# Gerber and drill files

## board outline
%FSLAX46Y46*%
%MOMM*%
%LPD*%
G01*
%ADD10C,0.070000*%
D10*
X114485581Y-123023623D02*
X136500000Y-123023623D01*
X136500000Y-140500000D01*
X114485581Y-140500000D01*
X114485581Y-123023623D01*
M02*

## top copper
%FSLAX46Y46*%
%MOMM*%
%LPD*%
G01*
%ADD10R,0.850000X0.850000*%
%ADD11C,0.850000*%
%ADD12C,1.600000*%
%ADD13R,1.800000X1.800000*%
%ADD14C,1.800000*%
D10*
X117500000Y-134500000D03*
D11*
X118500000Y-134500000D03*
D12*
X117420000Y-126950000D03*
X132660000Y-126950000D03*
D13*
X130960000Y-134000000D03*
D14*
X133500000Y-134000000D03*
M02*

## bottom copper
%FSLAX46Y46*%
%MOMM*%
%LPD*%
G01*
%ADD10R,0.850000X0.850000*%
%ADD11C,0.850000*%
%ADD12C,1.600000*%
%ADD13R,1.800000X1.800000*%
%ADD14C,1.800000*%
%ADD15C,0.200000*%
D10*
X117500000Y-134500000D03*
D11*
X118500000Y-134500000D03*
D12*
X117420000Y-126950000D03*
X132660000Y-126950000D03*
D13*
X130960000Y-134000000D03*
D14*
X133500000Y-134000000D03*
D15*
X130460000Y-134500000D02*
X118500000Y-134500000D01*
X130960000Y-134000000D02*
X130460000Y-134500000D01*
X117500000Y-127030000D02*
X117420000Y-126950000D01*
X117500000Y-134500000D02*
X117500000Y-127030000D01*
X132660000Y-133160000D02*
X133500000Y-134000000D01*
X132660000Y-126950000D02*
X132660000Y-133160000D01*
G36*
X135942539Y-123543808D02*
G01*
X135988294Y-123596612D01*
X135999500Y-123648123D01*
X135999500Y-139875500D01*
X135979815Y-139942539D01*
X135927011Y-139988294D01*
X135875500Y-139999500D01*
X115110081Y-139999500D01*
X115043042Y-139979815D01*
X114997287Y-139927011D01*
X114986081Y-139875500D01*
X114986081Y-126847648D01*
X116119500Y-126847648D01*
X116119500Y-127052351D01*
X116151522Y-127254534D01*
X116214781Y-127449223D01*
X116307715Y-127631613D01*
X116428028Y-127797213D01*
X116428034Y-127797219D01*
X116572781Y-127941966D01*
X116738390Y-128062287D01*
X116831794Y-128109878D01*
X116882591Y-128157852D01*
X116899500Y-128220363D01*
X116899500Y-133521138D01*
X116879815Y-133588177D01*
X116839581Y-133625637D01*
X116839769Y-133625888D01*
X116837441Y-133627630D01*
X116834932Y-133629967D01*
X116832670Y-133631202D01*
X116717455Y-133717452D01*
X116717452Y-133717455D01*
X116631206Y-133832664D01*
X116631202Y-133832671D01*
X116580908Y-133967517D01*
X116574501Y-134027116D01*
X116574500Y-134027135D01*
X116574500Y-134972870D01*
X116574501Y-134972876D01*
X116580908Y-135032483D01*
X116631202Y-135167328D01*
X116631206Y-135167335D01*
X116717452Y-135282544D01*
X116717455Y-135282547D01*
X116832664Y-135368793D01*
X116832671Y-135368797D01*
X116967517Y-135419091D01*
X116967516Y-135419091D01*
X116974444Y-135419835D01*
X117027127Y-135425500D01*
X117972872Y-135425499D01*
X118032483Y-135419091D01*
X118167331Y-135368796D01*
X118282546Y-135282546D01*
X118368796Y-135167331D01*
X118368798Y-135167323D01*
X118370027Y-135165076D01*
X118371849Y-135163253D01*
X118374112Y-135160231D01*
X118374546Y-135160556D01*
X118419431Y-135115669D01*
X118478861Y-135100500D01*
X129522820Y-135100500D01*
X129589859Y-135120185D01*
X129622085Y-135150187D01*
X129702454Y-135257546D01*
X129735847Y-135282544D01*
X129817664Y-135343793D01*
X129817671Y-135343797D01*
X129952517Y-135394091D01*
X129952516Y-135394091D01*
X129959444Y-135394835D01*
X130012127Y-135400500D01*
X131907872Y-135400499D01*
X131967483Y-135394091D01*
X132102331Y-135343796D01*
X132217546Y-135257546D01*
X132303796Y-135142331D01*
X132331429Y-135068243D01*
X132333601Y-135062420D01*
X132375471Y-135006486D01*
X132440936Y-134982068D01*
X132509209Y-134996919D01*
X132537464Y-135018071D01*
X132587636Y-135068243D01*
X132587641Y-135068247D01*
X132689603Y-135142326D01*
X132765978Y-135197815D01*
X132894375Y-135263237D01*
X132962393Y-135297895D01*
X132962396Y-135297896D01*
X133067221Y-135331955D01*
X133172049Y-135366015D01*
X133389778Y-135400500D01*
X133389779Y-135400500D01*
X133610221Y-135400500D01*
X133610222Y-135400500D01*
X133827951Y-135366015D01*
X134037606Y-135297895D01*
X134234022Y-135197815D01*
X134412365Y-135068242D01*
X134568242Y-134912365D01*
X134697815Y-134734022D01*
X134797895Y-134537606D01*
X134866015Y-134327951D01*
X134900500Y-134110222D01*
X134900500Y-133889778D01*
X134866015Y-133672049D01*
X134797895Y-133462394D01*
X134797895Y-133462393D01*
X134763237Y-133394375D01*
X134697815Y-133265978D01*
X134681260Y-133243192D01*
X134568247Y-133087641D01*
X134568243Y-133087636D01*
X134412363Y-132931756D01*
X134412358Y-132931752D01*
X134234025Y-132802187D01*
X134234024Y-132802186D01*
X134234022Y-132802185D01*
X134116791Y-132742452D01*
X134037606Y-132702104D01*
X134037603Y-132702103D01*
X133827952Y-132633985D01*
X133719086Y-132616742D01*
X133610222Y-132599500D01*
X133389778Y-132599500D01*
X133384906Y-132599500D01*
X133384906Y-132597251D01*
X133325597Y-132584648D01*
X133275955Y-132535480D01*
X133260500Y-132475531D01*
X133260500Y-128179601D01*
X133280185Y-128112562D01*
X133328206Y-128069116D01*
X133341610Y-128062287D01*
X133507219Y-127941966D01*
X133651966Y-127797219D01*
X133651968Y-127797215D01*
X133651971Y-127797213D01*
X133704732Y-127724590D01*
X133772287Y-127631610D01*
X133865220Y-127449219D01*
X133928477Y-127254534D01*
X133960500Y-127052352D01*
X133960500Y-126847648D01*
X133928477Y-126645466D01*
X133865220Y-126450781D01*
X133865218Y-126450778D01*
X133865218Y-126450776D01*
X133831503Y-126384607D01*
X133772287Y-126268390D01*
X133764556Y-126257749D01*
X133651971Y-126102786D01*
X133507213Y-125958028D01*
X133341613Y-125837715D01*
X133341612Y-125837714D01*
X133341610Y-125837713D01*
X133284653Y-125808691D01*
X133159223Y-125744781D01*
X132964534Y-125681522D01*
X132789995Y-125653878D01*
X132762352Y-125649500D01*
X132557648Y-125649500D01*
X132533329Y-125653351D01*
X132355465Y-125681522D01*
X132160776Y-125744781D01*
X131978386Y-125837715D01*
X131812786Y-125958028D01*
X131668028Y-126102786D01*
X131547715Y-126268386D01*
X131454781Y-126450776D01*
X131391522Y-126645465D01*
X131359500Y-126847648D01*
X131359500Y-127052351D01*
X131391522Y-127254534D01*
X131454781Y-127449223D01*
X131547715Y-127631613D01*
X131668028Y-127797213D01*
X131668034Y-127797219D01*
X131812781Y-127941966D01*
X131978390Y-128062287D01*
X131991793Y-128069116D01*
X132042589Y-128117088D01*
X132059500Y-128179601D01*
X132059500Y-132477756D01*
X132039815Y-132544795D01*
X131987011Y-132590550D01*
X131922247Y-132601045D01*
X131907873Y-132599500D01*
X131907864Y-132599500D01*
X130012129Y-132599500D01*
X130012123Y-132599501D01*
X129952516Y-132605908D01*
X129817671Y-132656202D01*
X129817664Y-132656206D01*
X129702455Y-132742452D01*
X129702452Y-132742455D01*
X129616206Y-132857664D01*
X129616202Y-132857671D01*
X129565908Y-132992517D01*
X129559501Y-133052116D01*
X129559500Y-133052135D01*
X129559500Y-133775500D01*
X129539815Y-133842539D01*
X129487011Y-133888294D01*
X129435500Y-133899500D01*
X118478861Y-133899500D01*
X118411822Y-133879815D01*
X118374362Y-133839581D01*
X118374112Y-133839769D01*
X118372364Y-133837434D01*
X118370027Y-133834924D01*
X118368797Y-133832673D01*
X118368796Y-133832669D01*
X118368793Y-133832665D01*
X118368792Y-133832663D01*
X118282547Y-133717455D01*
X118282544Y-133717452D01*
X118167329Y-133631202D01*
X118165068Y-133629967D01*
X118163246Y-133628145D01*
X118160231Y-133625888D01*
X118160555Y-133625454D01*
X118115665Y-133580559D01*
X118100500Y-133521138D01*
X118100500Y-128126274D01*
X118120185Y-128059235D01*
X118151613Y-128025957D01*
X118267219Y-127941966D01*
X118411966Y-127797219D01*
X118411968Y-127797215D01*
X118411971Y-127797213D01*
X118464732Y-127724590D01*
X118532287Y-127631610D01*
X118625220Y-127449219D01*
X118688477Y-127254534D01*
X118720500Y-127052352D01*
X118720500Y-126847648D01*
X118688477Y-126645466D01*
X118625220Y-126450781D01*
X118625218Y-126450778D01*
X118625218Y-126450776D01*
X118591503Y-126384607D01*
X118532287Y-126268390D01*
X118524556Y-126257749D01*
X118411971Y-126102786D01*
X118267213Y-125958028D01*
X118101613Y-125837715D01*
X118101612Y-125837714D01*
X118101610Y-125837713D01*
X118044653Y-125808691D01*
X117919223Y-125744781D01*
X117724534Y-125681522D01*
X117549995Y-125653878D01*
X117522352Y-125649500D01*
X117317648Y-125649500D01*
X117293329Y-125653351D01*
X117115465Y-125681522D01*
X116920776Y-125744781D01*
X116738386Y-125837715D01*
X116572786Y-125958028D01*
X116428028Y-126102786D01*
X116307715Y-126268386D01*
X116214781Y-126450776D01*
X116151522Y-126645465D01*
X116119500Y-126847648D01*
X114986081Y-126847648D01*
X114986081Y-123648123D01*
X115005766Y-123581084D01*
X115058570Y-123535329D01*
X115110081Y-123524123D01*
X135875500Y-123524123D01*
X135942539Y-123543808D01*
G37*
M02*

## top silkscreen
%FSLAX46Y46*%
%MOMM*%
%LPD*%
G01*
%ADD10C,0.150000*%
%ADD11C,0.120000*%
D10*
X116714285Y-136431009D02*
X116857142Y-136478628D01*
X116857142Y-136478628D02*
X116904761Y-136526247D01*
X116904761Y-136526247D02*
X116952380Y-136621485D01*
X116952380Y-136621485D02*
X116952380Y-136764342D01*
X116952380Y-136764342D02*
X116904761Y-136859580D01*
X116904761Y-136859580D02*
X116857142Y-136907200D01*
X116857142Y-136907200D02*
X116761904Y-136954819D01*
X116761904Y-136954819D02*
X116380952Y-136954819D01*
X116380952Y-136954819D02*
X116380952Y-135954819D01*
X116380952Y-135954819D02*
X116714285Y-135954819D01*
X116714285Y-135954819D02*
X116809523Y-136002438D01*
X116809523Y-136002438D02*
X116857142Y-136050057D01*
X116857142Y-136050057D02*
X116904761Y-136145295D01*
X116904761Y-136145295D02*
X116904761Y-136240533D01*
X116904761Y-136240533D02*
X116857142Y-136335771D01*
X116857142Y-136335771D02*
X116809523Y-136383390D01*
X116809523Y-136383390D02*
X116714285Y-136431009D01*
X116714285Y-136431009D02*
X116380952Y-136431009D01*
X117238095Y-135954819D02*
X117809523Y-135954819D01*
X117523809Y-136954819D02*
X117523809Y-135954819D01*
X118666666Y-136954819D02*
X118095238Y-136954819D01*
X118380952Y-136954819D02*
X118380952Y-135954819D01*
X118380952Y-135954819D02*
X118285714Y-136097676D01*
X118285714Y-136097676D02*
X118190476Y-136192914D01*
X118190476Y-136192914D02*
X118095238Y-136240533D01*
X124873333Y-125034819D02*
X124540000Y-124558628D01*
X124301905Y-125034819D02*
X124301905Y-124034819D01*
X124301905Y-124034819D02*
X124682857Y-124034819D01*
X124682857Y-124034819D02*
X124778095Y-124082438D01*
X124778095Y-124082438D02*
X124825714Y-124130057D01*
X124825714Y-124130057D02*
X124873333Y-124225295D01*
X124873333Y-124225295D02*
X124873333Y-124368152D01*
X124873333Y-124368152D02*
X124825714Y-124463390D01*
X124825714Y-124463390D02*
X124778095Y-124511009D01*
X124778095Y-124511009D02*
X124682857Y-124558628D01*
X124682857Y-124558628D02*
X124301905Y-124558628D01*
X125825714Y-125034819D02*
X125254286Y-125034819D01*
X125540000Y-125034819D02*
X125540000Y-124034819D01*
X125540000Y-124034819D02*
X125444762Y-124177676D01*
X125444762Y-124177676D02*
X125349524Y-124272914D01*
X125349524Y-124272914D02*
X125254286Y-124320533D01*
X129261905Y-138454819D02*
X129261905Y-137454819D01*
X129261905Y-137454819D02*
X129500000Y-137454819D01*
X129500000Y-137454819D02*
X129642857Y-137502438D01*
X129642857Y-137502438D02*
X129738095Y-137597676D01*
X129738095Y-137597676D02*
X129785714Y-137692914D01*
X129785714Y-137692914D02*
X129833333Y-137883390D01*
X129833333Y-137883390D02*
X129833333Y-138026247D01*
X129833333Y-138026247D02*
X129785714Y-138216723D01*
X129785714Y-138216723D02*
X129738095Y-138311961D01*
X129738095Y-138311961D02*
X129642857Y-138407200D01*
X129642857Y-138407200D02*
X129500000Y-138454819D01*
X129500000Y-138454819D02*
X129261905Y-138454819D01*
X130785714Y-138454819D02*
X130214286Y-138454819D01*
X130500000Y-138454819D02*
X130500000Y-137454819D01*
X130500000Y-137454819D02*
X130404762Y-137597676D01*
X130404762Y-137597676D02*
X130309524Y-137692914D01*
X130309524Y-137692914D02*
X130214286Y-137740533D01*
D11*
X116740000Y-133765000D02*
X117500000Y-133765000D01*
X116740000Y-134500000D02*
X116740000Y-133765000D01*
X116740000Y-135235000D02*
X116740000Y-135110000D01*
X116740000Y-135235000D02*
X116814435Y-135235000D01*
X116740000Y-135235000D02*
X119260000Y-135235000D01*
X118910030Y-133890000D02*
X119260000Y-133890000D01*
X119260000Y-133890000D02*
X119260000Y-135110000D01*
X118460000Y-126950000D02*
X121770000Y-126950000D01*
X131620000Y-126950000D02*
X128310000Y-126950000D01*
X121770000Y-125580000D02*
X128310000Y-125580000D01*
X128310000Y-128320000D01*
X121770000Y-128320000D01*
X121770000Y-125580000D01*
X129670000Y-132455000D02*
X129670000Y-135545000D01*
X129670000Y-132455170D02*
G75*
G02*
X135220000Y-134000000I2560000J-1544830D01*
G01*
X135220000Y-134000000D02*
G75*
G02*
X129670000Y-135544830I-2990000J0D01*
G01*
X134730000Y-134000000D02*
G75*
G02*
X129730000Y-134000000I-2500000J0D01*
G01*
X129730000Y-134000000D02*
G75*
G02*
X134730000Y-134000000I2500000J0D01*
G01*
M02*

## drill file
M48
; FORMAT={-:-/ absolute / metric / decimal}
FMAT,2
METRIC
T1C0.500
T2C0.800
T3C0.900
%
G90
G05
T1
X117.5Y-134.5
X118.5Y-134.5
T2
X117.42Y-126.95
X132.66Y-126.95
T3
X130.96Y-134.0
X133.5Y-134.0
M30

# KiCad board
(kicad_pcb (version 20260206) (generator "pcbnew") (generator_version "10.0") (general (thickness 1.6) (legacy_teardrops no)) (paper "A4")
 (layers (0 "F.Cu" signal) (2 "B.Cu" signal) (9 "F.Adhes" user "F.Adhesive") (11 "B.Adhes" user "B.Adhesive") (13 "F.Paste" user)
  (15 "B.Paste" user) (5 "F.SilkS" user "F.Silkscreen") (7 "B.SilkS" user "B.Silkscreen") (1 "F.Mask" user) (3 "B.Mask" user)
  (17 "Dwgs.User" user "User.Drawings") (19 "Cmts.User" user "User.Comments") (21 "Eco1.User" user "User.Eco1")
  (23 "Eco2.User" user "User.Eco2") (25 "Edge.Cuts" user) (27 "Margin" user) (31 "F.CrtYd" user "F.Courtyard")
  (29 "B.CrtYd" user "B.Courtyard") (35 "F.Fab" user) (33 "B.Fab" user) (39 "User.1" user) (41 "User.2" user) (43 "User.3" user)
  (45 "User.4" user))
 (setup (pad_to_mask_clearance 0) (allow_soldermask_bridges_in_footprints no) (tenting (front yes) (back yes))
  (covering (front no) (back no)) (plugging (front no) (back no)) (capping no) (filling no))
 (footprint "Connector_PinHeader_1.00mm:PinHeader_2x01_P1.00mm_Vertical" (layer "F.Cu") (at 117.5 134.5)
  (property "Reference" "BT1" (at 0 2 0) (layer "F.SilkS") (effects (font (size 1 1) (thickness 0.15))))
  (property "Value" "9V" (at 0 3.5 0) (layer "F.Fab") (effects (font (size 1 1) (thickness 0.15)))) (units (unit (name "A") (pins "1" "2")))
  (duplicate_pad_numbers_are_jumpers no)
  (fp_line (start -0.76 -0.735) (end 0 -0.735) (stroke (width 0.12) (type solid)) (layer "F.SilkS"))
  (fp_line (start -0.76 0) (end -0.76 -0.735) (stroke (width 0.12) (type solid)) (layer "F.SilkS"))
  (fp_line (start -0.76 0.735) (end -0.76 0.61) (stroke (width 0.12) (type solid)) (layer "F.SilkS"))
  (fp_line (start -0.76 0.735) (end -0.685565 0.735) (stroke (width 0.12) (type solid)) (layer "F.SilkS"))
  (fp_line (start -0.76 0.735) (end 1.76 0.735) (stroke (width 0.12) (type solid)) (layer "F.SilkS"))
  (fp_line (start 1.41003 -0.61) (end 1.76 -0.61) (stroke (width 0.12) (type solid)) (layer "F.SilkS"))
  (fp_line (start 1.76 -0.61) (end 1.76 0.61) (stroke (width 0.12) (type solid)) (layer "F.SilkS"))
  (pad "1" thru_hole rect (at 0 0) (size 0.85 0.85) (drill 0.5) (layers "*.Cu" "*.Mask") (remove_unused_layers no) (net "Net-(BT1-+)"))
  (pad "2" thru_hole circle (at 1 0) (size 0.85 0.85) (drill 0.5) (layers "*.Cu" "*.Mask") (remove_unused_layers no) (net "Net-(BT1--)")
   (clearance 0.15)))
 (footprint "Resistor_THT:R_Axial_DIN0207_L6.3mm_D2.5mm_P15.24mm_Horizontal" (layer "F.Cu") (at 117.42 126.95)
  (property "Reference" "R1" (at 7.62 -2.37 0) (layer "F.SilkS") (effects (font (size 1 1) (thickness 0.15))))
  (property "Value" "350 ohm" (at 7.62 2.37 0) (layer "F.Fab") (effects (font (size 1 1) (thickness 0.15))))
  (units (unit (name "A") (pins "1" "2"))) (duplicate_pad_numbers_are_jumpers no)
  (fp_line (start 1.04 0) (end 4.35 0) (stroke (width 0.12) (type solid)) (layer "F.SilkS"))
  (fp_line (start 14.2 0) (end 10.89 0) (stroke (width 0.12) (type solid)) (layer "F.SilkS"))
  (fp_rect (start 4.35 -1.37) (end 10.89 1.37) (stroke (width 0.12) (type solid)) (fill no) (layer "F.SilkS"))
  (pad "1" thru_hole circle (at 0 0) (size 1.6 1.6) (drill 0.8) (layers "*.Cu" "*.Mask") (remove_unused_layers no) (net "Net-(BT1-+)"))
  (pad "2" thru_hole circle (at 15.24 0) (size 1.6 1.6) (drill 0.8) (layers "*.Cu" "*.Mask") (remove_unused_layers no) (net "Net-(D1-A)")))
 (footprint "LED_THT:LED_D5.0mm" (layer "F.Cu") (at 130.96 134)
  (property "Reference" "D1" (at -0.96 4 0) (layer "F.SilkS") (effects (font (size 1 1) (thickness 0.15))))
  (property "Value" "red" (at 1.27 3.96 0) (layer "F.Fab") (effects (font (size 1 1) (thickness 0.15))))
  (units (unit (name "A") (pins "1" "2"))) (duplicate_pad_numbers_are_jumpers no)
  (fp_line (start -1.29 -1.545) (end -1.29 1.545) (stroke (width 0.12) (type solid)) (layer "F.SilkS"))
  (fp_arc (start -1.29 -1.54483) (mid 2.071779 -2.880495) (end 4.26 0) (stroke (width 0.12) (type solid)) (layer "F.SilkS"))
  (fp_arc (start 4.26 0) (mid 2.071779 2.880495) (end -1.29 1.54483) (stroke (width 0.12) (type solid)) (layer "F.SilkS"))
  (fp_circle (center 1.27 0) (end 3.77 0) (stroke (width 0.12) (type solid)) (fill no) (layer "F.SilkS"))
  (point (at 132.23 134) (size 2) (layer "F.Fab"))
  (pad "1" thru_hole rect (at 0 0) (size 1.8 1.8) (drill 0.9) (layers "*.Cu" "*.Mask") (remove_unused_layers no) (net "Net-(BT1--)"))
  (pad "2" thru_hole circle (at 2.54 0) (size 1.8 1.8) (drill 0.9) (layers "*.Cu" "*.Mask") (remove_unused_layers no) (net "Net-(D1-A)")))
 (gr_rect (start 114.485581 123.023623) (end 136.5 140.5) (stroke (width 0.07) (type solid)) (fill no) (layer "Edge.Cuts"))
 (segment (start 130.46 134.5) (end 118.5 134.5) (width 0.2) (layer "B.Cu") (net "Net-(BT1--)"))
 (segment (start 130.96 134) (end 130.46 134.5) (width 0.2) (layer "B.Cu") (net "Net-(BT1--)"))
 (segment (start 117.5 127.03) (end 117.42 126.95) (width 0.2) (layer "B.Cu") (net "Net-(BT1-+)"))
 (segment (start 117.5 134.5) (end 117.5 127.03) (width 0.2) (layer "B.Cu") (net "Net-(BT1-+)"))
 (segment (start 132.66 133.16) (end 133.5 134) (width 0.2) (layer "B.Cu") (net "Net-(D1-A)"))
 (segment (start 132.66 126.95) (end 132.66 133.16) (width 0.2) (layer "B.Cu") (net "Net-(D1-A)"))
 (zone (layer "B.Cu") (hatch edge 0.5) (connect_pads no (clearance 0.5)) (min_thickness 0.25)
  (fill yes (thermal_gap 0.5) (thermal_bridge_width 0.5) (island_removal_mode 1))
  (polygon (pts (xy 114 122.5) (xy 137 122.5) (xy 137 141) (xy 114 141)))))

